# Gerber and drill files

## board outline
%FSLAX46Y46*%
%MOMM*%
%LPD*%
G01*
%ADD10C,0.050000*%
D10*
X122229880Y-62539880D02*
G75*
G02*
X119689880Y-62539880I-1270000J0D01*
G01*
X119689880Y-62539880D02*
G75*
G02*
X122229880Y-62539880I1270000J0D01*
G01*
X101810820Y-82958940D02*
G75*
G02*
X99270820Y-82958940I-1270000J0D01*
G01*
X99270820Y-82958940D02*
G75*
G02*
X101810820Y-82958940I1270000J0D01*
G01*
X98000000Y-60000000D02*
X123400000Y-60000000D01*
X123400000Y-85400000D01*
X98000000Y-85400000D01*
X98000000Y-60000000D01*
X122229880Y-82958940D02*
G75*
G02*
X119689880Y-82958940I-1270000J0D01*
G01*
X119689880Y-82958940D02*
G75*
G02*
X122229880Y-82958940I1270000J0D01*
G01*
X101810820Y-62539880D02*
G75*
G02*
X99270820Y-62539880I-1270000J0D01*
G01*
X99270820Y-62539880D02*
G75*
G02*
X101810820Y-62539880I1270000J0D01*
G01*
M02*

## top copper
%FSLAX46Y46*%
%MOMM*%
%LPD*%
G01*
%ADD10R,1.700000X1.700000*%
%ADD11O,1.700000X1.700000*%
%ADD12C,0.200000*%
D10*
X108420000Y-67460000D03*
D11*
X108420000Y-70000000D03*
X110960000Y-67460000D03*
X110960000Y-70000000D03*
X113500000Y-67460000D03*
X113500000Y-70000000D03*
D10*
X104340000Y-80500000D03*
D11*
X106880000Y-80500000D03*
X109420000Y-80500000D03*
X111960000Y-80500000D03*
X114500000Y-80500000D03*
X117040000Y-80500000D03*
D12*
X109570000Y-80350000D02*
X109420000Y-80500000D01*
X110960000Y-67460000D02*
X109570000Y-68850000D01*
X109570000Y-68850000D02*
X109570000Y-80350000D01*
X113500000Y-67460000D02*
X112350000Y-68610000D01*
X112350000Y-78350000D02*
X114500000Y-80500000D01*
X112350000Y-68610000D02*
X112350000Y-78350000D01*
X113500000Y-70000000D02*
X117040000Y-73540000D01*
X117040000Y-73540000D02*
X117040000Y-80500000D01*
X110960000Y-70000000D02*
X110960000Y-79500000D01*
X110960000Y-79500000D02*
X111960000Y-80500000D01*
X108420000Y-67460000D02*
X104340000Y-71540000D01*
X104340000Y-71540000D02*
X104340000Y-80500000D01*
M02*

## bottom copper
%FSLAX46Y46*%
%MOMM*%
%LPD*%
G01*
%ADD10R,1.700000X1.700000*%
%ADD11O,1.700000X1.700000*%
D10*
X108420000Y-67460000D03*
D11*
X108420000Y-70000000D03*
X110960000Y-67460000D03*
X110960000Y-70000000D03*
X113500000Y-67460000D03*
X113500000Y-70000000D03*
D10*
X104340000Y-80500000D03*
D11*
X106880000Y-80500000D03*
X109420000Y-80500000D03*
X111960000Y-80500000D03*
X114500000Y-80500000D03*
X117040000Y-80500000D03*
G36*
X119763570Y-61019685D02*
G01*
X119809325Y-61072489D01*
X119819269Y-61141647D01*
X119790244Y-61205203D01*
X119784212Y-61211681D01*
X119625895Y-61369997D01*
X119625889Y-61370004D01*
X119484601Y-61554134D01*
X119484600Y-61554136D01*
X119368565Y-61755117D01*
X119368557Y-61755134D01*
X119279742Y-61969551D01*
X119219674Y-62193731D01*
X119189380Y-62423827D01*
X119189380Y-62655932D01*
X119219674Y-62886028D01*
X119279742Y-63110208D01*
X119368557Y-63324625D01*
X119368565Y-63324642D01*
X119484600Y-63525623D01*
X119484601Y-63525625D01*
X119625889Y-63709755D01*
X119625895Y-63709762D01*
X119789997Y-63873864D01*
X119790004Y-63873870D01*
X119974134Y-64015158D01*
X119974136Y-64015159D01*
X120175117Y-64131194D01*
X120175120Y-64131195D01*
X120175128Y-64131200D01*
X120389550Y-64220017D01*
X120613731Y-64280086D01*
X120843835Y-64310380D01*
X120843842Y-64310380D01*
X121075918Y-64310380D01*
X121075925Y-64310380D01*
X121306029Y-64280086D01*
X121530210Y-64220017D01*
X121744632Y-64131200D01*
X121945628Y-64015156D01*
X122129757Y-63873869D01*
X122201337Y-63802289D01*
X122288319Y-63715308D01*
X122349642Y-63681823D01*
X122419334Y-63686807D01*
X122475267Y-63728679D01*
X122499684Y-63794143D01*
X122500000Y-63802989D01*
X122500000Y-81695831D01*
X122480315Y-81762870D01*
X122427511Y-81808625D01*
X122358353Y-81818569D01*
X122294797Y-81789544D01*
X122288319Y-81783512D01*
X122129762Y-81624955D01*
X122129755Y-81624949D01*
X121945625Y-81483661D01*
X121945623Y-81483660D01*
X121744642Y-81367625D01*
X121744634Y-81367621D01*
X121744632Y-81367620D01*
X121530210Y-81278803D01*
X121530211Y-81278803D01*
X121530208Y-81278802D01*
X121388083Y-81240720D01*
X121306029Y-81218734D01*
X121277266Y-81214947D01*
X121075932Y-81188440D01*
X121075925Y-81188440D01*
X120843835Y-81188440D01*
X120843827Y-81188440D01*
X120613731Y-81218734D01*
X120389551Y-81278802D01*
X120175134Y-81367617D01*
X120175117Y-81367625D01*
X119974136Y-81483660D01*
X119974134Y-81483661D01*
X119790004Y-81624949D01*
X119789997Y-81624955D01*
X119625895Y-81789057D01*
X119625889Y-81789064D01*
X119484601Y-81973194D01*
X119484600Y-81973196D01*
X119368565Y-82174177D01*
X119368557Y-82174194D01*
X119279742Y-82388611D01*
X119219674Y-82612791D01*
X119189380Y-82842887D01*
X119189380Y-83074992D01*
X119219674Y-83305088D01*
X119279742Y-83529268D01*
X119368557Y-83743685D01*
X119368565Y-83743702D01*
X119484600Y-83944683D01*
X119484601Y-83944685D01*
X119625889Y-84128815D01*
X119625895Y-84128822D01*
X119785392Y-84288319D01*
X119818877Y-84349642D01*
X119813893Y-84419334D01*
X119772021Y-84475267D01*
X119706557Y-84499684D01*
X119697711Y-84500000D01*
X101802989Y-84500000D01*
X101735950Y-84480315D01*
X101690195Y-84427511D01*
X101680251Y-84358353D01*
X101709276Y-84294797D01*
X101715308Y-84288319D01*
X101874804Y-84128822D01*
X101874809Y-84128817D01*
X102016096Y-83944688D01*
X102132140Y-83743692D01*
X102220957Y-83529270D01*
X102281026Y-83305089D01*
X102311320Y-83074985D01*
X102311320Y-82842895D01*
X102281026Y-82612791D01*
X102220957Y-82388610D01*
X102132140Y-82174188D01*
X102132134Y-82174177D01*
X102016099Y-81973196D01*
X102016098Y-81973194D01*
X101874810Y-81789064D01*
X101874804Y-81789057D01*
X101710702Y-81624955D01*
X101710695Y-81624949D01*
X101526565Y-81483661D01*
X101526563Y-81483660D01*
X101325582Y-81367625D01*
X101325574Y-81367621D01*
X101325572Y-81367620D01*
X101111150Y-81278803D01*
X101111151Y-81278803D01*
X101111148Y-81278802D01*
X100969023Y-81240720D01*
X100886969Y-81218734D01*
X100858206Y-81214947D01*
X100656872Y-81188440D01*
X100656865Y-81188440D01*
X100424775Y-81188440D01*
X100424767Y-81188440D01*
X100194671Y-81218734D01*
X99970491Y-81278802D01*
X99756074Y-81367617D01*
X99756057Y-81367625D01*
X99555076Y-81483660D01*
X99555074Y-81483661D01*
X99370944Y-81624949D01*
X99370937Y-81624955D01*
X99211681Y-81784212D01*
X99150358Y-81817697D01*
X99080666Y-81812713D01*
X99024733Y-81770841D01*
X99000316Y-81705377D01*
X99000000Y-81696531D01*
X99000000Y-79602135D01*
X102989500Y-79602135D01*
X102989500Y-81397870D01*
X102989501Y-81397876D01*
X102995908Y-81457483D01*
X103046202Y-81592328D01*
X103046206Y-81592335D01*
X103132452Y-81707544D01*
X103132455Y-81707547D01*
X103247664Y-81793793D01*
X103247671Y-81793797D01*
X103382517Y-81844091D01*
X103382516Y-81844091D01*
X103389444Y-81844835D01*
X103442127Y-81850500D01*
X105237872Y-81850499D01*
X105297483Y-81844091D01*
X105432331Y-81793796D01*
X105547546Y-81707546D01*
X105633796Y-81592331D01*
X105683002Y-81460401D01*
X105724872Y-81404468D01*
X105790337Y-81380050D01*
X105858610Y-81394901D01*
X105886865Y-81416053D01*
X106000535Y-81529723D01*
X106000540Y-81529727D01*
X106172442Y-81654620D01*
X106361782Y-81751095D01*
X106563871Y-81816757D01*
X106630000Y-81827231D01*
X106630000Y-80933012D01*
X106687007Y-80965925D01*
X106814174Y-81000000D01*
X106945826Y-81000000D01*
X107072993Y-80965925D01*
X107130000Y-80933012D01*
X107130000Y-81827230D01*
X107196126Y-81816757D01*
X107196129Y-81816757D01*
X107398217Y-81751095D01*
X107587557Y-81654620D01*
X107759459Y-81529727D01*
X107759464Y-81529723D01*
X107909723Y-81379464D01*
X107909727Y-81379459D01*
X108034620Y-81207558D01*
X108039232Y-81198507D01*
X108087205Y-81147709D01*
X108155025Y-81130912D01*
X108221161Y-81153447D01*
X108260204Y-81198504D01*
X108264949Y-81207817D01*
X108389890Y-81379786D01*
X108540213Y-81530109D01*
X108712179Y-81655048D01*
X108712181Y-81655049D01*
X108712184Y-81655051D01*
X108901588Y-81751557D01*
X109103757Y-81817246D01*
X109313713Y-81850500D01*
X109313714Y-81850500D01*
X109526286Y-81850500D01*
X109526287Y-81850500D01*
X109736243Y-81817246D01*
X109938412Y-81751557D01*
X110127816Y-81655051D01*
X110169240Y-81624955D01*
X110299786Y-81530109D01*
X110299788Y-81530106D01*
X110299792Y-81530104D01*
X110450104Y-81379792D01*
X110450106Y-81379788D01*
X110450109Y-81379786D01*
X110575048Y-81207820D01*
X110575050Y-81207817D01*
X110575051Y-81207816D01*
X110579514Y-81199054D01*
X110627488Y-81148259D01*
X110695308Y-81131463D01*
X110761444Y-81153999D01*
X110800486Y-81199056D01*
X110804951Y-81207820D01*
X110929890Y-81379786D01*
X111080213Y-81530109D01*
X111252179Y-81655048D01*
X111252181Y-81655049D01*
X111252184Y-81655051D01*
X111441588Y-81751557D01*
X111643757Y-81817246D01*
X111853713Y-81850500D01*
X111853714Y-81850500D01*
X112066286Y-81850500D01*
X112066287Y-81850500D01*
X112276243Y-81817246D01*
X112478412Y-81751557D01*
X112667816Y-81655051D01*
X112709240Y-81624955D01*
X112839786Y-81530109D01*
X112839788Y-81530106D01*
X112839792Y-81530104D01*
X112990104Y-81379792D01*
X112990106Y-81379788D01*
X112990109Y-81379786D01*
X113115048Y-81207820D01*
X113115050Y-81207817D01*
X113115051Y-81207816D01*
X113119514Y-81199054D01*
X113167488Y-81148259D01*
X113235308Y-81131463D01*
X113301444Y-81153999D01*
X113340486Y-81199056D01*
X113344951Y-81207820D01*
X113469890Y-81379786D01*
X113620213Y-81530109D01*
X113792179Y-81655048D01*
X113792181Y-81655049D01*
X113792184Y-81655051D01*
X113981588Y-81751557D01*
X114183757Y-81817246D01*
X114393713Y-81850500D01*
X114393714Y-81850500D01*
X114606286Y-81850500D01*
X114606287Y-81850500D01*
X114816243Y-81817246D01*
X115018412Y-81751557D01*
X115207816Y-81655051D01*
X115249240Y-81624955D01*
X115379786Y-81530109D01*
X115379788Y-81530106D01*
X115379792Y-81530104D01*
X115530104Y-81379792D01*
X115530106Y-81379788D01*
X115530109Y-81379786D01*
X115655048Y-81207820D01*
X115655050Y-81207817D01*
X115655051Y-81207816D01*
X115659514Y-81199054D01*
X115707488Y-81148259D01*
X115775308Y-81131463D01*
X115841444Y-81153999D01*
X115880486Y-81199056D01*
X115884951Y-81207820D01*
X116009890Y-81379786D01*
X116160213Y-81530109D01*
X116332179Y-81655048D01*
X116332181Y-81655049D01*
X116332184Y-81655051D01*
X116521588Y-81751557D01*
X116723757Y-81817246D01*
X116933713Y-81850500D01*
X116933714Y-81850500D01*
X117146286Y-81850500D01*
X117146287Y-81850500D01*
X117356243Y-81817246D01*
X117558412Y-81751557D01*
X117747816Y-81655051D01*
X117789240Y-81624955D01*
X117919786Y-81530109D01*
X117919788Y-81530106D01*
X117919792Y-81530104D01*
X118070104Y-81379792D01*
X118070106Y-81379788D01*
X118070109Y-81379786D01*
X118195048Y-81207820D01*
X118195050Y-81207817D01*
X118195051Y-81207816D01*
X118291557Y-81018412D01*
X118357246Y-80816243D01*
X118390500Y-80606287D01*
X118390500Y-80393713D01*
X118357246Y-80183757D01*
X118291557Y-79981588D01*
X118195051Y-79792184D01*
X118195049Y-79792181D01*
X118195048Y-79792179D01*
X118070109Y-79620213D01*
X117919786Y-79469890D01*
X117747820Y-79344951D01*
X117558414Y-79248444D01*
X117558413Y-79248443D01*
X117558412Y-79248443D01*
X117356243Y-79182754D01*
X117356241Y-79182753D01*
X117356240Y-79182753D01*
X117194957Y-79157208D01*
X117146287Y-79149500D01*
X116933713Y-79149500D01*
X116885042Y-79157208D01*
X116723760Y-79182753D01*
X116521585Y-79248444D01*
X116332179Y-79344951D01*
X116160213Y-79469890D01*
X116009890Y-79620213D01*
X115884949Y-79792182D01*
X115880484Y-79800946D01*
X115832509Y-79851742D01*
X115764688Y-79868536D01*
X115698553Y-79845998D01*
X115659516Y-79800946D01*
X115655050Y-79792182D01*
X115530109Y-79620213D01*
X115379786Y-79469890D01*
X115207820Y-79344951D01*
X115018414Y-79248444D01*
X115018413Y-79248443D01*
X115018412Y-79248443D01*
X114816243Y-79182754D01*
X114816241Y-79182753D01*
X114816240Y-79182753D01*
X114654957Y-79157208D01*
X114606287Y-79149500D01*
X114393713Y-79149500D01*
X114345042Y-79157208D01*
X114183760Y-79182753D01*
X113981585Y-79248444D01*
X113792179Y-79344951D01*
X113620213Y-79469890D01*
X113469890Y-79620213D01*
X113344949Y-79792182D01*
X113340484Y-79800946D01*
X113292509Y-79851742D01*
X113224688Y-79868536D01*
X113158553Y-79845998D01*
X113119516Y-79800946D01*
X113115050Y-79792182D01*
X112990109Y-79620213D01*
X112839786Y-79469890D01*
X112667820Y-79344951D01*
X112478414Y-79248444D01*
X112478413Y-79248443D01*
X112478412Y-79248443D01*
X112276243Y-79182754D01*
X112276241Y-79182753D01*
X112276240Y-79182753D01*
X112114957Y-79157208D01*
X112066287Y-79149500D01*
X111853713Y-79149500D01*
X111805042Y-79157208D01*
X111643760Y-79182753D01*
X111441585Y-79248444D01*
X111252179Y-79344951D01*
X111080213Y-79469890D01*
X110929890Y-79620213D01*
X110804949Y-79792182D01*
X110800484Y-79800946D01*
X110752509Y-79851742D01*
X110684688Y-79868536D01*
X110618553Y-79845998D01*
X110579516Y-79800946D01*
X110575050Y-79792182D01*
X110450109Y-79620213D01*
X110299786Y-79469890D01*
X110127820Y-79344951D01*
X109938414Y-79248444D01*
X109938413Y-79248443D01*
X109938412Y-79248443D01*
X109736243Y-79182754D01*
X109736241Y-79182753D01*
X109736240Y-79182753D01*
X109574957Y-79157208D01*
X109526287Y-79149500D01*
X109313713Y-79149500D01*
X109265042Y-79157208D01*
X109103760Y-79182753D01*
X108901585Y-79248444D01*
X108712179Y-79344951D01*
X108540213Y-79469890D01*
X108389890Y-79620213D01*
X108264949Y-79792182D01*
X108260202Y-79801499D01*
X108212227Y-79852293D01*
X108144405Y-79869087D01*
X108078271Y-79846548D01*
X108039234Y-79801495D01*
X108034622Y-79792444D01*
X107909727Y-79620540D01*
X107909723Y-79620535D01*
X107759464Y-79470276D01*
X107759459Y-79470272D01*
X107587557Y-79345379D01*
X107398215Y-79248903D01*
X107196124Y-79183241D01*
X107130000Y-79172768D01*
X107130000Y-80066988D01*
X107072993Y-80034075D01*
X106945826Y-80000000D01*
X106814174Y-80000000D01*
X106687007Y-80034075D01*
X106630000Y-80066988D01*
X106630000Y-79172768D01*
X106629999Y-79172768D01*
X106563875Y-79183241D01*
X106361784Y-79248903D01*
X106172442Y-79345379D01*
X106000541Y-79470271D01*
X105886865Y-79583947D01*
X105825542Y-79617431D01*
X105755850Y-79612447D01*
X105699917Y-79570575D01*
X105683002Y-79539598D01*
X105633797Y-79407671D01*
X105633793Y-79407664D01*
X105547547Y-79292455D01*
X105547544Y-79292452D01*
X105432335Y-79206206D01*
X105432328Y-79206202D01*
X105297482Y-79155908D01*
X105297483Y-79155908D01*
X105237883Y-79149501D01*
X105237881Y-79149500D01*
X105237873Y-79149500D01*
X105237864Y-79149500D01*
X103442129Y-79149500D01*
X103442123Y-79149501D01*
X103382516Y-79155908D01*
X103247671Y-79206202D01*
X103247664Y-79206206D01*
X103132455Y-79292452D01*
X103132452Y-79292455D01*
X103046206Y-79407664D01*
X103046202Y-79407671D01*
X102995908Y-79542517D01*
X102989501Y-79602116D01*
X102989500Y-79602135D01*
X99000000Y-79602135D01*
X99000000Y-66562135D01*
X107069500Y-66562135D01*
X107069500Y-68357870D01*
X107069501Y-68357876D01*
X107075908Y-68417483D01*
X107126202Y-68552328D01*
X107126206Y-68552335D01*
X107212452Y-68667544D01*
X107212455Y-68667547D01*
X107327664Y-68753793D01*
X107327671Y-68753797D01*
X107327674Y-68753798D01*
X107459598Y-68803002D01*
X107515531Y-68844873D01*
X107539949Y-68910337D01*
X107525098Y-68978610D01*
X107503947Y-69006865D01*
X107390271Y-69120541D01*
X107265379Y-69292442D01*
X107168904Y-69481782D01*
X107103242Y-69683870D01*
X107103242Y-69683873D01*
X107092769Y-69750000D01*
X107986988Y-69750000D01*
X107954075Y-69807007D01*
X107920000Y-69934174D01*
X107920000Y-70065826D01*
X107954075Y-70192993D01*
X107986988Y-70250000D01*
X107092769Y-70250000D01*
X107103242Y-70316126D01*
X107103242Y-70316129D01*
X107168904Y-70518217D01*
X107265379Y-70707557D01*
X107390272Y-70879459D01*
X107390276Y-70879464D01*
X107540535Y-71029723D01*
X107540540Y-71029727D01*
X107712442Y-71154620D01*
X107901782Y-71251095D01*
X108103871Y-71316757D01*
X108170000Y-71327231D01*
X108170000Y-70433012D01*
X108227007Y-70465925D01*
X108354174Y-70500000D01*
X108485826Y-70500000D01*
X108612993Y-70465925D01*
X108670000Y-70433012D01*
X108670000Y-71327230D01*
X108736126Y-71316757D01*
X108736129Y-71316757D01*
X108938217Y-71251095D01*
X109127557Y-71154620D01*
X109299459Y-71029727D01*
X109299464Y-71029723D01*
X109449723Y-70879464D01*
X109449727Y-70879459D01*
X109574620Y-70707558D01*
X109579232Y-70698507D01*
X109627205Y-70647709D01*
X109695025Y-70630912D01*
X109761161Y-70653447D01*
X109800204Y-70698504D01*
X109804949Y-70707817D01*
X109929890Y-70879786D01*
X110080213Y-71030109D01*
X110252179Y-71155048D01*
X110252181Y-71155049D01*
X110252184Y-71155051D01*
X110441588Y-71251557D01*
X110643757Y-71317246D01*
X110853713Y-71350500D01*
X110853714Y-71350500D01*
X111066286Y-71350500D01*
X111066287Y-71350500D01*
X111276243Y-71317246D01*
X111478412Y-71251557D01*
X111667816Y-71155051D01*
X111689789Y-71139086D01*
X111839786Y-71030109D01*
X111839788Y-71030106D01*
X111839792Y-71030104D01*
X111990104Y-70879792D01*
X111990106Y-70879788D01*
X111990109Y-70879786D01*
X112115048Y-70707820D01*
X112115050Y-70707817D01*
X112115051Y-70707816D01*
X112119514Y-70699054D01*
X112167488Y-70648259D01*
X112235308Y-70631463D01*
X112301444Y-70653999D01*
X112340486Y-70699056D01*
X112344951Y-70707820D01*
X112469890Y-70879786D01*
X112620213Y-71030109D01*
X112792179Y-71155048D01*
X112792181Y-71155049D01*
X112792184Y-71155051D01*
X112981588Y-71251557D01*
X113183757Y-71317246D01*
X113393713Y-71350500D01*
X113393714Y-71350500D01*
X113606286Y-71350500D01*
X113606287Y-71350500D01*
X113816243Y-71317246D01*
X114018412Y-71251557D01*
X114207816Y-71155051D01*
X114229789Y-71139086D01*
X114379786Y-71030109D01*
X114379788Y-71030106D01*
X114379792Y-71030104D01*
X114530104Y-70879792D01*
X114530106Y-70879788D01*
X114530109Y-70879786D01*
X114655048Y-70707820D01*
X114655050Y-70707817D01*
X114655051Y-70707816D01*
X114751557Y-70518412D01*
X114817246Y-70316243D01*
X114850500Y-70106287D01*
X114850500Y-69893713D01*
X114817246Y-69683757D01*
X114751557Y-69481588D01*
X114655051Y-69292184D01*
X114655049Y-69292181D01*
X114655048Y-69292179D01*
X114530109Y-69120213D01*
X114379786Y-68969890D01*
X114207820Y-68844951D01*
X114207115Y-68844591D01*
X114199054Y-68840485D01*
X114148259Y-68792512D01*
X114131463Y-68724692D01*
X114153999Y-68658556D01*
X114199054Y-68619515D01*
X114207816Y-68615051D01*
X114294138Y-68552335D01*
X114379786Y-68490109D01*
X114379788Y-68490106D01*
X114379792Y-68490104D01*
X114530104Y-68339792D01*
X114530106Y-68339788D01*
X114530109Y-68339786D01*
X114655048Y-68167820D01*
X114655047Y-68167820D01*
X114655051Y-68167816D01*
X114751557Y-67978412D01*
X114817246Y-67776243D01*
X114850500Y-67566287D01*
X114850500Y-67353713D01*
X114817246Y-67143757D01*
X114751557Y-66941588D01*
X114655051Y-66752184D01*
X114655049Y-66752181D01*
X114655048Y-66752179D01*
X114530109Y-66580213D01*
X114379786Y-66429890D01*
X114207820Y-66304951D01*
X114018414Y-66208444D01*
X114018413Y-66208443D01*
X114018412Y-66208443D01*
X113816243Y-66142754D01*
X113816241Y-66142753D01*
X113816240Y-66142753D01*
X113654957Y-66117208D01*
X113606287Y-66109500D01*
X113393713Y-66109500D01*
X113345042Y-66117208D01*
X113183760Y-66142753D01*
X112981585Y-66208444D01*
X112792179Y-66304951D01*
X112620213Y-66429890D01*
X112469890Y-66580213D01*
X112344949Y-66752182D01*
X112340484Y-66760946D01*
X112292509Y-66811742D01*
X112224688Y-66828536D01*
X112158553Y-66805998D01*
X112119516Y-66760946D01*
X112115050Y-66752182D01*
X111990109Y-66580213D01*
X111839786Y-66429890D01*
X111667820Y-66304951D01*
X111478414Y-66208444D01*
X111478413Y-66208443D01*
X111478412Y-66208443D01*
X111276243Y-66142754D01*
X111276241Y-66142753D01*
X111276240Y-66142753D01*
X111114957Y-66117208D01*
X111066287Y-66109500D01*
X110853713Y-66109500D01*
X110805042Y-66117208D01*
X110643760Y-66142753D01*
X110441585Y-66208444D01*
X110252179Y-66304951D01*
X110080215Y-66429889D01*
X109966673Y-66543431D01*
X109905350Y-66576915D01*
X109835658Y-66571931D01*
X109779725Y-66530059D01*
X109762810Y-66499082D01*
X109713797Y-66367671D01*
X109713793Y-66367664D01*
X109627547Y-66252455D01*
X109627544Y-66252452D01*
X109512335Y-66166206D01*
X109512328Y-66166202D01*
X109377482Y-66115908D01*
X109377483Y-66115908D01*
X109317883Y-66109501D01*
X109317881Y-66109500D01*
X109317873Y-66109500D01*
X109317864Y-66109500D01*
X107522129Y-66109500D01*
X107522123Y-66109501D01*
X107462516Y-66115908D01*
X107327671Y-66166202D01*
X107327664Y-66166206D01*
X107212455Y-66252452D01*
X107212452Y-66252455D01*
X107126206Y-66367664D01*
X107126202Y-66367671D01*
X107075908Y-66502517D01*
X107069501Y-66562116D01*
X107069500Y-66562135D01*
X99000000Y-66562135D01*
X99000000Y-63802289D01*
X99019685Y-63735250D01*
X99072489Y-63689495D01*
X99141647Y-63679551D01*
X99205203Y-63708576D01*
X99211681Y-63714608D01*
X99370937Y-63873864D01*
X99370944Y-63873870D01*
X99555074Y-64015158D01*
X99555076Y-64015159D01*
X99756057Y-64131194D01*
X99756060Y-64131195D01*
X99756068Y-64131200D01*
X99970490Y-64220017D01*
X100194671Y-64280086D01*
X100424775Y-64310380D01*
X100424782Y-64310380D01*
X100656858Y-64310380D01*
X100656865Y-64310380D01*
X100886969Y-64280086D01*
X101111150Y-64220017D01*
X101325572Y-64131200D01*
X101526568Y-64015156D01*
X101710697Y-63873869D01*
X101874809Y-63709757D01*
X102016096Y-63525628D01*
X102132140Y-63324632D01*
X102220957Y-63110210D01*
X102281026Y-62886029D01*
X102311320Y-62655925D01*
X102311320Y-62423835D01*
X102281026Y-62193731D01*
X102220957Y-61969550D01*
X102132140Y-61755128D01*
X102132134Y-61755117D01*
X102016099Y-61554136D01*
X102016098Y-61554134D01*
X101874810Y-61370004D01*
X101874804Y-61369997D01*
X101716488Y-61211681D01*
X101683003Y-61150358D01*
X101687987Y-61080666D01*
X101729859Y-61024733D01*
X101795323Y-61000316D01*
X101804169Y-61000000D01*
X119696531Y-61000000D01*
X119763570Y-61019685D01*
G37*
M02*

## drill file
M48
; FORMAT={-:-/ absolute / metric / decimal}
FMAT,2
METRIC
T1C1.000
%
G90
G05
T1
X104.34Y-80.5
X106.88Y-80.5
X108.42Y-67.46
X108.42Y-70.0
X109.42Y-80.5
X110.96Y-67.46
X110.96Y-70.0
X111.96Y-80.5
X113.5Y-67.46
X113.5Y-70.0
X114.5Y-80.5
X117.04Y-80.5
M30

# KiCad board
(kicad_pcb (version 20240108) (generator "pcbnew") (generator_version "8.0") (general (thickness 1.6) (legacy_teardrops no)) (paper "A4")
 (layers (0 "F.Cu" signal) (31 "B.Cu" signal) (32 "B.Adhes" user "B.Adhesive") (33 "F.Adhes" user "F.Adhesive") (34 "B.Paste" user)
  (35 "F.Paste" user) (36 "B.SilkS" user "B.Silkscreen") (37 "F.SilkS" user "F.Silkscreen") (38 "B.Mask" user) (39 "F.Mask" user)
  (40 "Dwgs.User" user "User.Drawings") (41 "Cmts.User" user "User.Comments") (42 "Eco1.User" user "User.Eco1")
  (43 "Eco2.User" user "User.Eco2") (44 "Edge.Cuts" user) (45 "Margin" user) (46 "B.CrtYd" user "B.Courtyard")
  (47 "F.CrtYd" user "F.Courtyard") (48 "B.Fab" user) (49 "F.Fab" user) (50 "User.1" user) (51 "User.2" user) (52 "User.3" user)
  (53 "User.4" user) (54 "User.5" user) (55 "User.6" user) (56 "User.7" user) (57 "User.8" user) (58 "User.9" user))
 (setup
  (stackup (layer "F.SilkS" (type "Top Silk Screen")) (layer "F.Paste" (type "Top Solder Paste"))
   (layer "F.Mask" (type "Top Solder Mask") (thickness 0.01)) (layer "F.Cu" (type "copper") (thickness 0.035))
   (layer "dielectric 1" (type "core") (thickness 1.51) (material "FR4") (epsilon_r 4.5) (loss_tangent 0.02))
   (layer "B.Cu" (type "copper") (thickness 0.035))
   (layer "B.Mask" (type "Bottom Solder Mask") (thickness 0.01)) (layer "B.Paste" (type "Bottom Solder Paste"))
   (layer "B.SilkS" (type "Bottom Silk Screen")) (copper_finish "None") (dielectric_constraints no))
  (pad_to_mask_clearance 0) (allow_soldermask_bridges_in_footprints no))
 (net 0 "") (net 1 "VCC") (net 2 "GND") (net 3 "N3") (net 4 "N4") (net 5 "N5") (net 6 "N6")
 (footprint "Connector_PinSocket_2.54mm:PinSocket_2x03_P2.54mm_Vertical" (layer "F.Cu") (at 108.42 67.46 90)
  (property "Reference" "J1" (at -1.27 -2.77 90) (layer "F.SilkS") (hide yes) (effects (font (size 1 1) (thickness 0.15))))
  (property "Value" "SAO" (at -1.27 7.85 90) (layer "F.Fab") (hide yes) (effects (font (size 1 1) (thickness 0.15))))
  (pad "1" thru_hole rect (at 0 0 90) (size 1.7 1.7) (drill 1) (layers "*.Cu" "*.Mask") (remove_unused_layers no) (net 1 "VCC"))
  (pad "2" thru_hole oval (at -2.54 0 90) (size 1.7 1.7) (drill 1) (layers "*.Cu" "*.Mask") (remove_unused_layers no) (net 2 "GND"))
  (pad "3" thru_hole oval (at 0 2.54 90) (size 1.7 1.7) (drill 1) (layers "*.Cu" "*.Mask") (remove_unused_layers no) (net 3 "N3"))
  (pad "4" thru_hole oval (at -2.54 2.54 90) (size 1.7 1.7) (drill 1) (layers "*.Cu" "*.Mask") (remove_unused_layers no) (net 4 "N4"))
  (pad "5" thru_hole oval (at 0 5.08 90) (size 1.7 1.7) (drill 1) (layers "*.Cu" "*.Mask") (remove_unused_layers no) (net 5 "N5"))
  (pad "6" thru_hole oval (at -2.54 5.08 90) (size 1.7 1.7) (drill 1) (layers "*.Cu" "*.Mask") (remove_unused_layers no) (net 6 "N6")))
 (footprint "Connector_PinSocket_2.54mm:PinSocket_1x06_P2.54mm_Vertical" (layer "F.Cu") (at 104.34 80.5 90)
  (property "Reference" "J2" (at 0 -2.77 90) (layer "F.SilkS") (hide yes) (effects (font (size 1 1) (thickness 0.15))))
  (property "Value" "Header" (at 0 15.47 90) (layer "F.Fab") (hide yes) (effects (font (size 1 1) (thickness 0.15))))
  (pad "1" thru_hole rect (at 0 0 90) (size 1.7 1.7) (drill 1) (layers "*.Cu" "*.Mask") (remove_unused_layers no) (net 1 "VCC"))
  (pad "2" thru_hole oval (at 0 2.54 90) (size 1.7 1.7) (drill 1) (layers "*.Cu" "*.Mask") (remove_unused_layers no) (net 2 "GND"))
  (pad "3" thru_hole oval (at 0 5.08 90) (size 1.7 1.7) (drill 1) (layers "*.Cu" "*.Mask") (remove_unused_layers no) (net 3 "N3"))
  (pad "4" thru_hole oval (at 0 7.62 90) (size 1.7 1.7) (drill 1) (layers "*.Cu" "*.Mask") (remove_unused_layers no) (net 4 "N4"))
  (pad "5" thru_hole oval (at 0 10.16 90) (size 1.7 1.7) (drill 1) (layers "*.Cu" "*.Mask") (remove_unused_layers no) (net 5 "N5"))
  (pad "6" thru_hole oval (at 0 12.7 90) (size 1.7 1.7) (drill 1) (layers "*.Cu" "*.Mask") (remove_unused_layers no) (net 6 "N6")))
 (gr_circle (center 120.95988 62.53988) (end 122.22988 62.53988) (stroke (width 0.05) (type default)) (fill none) (layer "Edge.Cuts"))
 (gr_circle (center 100.54082 82.95894) (end 101.81082 82.95894) (stroke (width 0.05) (type default)) (fill none) (layer "Edge.Cuts"))
 (gr_rect (start 98 60) (end 123.4 85.4) (stroke (width 0.05) (type default)) (fill none) (layer "Edge.Cuts"))
 (gr_circle (center 120.95988 82.95894) (end 122.22988 82.95894) (stroke (width 0.05) (type default)) (fill none) (layer "Edge.Cuts"))
 (gr_circle (center 100.54082 62.53988) (end 101.81082 62.53988) (stroke (width 0.05) (type default)) (fill none) (layer "Edge.Cuts"))
 (segment (start 109.57 80.35) (end 109.42 80.5) (width 0.2) (layer "F.Cu") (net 3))
 (segment (start 110.96 67.46) (end 109.57 68.85) (width 0.2) (layer "F.Cu") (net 3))
 (segment (start 109.57 68.85) (end 109.57 80.35) (width 0.2) (layer "F.Cu") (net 3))
 (segment (start 113.5 67.46) (end 112.35 68.61) (width 0.2) (layer "F.Cu") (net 5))
 (segment (start 112.35 78.35) (end 114.5 80.5) (width 0.2) (layer "F.Cu") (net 5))
 (segment (start 112.35 68.61) (end 112.35 78.35) (width 0.2) (layer "F.Cu") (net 5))
 (segment (start 113.5 70) (end 117.04 73.54) (width 0.2) (layer "F.Cu") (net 6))
 (segment (start 117.04 73.54) (end 117.04 80.5) (width 0.2) (layer "F.Cu") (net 6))
 (segment (start 110.96 70) (end 110.96 79.5) (width 0.2) (layer "F.Cu") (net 4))
 (segment (start 110.96 79.5) (end 111.96 80.5) (width 0.2) (layer "F.Cu") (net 4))
 (segment (start 108.42 67.46) (end 104.34 71.54) (width 0.2) (layer "F.Cu") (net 1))
 (segment (start 104.34 71.54) (end 104.34 80.5) (width 0.2) (layer "F.Cu") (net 1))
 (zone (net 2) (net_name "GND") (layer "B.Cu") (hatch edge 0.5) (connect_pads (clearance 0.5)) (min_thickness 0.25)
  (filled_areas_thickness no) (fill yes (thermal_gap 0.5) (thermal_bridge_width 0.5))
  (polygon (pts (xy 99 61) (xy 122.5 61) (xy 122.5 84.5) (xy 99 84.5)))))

